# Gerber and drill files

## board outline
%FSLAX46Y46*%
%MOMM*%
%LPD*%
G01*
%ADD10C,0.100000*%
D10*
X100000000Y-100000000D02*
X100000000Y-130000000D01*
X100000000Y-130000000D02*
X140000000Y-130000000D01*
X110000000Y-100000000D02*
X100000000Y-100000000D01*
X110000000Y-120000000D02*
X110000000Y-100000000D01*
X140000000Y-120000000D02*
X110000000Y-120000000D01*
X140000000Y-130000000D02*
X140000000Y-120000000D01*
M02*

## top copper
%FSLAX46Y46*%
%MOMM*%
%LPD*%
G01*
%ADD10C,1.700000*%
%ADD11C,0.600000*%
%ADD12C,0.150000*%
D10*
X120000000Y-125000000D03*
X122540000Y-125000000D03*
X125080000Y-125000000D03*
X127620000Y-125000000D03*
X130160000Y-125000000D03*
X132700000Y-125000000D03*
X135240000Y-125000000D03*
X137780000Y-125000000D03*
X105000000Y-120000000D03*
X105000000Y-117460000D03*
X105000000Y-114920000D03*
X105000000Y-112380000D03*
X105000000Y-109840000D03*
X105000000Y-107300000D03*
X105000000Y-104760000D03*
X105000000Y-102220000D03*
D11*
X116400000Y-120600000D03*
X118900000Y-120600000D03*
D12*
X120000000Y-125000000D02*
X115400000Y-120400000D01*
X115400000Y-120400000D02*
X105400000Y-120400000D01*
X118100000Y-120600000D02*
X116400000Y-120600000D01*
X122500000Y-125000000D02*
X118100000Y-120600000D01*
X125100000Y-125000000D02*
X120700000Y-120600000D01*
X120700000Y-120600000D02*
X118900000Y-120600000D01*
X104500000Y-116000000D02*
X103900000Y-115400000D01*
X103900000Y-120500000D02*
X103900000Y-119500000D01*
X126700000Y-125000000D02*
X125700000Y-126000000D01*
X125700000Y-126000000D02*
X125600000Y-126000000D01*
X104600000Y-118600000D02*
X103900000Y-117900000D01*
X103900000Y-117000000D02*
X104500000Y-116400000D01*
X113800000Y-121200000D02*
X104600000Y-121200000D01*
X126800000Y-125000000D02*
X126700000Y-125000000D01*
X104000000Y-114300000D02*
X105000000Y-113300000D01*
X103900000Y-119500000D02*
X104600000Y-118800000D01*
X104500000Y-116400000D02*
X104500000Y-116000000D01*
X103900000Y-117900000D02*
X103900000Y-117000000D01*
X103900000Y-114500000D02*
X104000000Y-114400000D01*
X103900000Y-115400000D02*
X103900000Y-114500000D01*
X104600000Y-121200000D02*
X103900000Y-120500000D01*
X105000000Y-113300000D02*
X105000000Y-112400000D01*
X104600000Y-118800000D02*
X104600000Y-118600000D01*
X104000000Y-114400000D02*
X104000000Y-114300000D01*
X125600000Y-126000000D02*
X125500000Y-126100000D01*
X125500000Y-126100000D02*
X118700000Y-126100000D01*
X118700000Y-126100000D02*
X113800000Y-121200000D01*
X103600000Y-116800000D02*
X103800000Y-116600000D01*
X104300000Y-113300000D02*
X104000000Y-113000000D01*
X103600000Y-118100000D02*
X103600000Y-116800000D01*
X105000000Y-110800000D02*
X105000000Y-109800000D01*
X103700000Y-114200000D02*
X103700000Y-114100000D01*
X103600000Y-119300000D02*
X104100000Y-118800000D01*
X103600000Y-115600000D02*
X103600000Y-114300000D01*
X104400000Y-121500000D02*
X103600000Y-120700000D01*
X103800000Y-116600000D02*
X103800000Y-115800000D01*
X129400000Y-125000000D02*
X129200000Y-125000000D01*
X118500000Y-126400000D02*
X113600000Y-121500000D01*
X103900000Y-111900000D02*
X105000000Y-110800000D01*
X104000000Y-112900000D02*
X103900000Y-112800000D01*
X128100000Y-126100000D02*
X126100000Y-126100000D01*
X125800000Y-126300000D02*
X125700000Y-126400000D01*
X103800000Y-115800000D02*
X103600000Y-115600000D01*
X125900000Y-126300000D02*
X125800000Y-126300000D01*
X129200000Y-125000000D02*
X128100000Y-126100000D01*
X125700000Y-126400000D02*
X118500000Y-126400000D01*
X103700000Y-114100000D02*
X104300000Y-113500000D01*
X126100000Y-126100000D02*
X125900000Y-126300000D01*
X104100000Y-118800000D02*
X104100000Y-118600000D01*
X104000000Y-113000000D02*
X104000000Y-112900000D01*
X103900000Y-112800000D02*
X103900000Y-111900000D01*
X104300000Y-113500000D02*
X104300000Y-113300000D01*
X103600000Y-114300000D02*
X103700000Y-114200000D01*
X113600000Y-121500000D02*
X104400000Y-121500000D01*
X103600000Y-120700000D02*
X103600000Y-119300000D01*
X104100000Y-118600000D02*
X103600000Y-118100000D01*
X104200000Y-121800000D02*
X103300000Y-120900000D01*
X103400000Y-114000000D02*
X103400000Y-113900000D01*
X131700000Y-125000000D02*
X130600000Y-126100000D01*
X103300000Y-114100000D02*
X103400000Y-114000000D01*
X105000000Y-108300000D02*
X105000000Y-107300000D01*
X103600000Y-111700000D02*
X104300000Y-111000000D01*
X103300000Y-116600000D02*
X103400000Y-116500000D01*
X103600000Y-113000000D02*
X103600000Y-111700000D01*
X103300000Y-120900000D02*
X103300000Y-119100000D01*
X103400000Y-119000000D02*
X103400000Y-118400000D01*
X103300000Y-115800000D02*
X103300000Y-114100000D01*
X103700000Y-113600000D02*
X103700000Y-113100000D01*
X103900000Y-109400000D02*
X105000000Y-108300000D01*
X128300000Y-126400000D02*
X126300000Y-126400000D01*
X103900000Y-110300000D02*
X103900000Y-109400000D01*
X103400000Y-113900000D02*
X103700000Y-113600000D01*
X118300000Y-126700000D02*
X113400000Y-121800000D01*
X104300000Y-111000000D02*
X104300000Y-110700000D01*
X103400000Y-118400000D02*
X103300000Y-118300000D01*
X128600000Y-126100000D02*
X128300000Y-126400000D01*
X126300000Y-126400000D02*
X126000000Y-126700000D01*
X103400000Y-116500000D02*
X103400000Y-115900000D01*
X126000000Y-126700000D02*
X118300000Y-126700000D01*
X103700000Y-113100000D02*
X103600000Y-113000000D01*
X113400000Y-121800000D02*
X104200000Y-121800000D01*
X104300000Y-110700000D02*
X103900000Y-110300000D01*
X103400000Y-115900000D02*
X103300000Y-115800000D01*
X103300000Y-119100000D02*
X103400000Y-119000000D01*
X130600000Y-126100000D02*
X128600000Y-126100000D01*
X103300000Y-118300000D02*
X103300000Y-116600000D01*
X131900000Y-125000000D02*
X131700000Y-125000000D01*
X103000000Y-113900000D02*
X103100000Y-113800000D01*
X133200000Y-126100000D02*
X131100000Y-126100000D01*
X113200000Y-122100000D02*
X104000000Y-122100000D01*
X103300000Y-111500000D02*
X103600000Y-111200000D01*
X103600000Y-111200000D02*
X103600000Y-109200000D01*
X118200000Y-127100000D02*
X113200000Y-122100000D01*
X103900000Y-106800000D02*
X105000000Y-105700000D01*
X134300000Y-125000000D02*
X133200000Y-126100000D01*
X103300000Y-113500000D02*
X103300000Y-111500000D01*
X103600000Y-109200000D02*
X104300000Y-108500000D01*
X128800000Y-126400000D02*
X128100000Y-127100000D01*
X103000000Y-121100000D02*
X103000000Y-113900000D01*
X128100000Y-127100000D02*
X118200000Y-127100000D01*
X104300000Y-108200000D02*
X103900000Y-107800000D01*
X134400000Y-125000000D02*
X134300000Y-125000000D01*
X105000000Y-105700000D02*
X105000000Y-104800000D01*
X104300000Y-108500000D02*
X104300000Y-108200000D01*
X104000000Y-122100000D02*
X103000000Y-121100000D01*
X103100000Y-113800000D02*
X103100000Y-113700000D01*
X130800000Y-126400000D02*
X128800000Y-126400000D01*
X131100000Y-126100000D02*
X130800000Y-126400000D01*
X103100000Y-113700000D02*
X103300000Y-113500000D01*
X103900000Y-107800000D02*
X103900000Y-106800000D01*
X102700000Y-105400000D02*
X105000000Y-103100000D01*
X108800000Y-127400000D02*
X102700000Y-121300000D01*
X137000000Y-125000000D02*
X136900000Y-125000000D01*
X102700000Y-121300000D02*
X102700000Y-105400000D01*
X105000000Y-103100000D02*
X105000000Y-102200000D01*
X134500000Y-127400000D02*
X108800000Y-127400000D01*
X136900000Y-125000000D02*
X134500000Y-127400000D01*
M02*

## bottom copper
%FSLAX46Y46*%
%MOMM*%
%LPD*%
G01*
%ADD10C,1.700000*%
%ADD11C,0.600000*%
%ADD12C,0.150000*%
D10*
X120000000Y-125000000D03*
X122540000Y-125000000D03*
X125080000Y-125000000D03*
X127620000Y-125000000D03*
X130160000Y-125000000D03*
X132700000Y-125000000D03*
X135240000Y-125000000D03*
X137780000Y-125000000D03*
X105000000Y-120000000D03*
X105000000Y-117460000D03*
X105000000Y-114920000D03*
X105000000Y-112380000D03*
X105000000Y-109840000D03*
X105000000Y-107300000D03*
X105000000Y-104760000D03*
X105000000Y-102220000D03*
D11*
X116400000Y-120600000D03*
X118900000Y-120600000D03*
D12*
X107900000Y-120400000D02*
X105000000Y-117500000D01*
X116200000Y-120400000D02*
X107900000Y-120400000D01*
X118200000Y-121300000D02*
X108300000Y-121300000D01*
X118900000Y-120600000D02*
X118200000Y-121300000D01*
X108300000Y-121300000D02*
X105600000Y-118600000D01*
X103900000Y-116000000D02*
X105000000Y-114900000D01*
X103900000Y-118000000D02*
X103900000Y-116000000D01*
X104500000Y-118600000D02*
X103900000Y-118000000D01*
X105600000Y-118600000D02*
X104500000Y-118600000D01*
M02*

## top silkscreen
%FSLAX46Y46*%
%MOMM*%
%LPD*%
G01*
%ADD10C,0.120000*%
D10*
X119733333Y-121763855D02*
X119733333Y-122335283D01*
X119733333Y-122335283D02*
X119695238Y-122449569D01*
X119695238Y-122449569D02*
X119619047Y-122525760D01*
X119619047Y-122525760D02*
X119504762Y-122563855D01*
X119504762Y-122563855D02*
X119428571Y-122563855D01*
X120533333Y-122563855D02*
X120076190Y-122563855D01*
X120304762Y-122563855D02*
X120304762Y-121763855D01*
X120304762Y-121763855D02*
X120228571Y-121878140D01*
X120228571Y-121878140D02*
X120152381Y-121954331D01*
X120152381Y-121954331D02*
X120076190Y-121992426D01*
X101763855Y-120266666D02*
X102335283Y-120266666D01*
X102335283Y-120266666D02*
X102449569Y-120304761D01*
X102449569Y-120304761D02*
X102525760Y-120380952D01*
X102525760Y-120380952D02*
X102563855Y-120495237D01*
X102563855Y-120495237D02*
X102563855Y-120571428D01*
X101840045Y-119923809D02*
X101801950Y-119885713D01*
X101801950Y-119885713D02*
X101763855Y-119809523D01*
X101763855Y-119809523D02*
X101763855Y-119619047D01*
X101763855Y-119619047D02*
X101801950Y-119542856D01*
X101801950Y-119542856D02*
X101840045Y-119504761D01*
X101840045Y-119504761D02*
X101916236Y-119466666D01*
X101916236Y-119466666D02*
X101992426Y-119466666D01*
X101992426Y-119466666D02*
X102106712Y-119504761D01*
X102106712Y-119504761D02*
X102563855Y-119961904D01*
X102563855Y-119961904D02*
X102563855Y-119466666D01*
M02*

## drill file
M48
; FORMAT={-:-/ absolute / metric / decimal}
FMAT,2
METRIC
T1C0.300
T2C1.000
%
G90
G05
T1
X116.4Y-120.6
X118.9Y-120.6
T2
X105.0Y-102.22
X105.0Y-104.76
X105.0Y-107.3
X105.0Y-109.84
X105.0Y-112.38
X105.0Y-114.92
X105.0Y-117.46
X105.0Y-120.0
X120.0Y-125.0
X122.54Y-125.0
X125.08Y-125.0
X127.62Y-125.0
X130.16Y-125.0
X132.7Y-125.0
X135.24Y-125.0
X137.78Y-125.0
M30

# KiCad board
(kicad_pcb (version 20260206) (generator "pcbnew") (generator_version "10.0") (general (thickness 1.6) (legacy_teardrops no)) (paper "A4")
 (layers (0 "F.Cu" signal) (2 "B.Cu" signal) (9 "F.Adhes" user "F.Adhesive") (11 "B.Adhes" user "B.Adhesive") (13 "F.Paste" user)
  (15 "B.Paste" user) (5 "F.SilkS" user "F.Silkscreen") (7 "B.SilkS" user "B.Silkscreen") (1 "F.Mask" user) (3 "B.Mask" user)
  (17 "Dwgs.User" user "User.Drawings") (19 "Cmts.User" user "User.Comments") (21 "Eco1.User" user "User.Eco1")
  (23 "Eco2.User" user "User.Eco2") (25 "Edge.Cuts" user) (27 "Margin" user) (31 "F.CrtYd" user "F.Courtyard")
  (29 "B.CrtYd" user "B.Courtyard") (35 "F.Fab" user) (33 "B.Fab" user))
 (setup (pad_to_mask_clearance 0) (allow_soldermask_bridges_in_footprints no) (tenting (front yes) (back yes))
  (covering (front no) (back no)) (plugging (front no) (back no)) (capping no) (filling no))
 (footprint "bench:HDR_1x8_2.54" (layer "F.Cu") (at 120 125)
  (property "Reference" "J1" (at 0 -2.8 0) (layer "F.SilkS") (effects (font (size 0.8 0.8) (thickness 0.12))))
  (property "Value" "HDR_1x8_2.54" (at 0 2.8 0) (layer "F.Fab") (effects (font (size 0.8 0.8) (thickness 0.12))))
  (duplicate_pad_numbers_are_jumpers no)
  (pad "1" thru_hole circle (at 0 0) (size 1.7 1.7) (drill 1) (layers "*.Cu" "*.Mask") (remove_unused_layers no) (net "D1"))
  (pad "2" thru_hole circle (at 2.54 0) (size 1.7 1.7) (drill 1) (layers "*.Cu" "*.Mask") (remove_unused_layers no) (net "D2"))
  (pad "3" thru_hole circle (at 5.08 0) (size 1.7 1.7) (drill 1) (layers "*.Cu" "*.Mask") (remove_unused_layers no) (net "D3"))
  (pad "4" thru_hole circle (at 7.62 0) (size 1.7 1.7) (drill 1) (layers "*.Cu" "*.Mask") (remove_unused_layers no) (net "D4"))
  (pad "5" thru_hole circle (at 10.16 0) (size 1.7 1.7) (drill 1) (layers "*.Cu" "*.Mask") (remove_unused_layers no) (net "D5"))
  (pad "6" thru_hole circle (at 12.7 0) (size 1.7 1.7) (drill 1) (layers "*.Cu" "*.Mask") (remove_unused_layers no) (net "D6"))
  (pad "7" thru_hole circle (at 15.24 0) (size 1.7 1.7) (drill 1) (layers "*.Cu" "*.Mask") (remove_unused_layers no) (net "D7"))
  (pad "8" thru_hole circle (at 17.78 0) (size 1.7 1.7) (drill 1) (layers "*.Cu" "*.Mask") (remove_unused_layers no) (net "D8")))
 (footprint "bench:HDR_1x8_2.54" (layer "F.Cu") (at 105 120 90)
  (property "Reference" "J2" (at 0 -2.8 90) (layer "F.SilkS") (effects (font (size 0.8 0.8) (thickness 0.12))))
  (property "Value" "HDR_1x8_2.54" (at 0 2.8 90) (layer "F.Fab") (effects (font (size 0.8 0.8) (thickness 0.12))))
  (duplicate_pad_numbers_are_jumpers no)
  (pad "1" thru_hole circle (at 0 0 90) (size 1.7 1.7) (drill 1) (layers "*.Cu" "*.Mask") (remove_unused_layers no) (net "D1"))
  (pad "2" thru_hole circle (at 2.54 0 90) (size 1.7 1.7) (drill 1) (layers "*.Cu" "*.Mask") (remove_unused_layers no) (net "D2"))
  (pad "3" thru_hole circle (at 5.08 0 90) (size 1.7 1.7) (drill 1) (layers "*.Cu" "*.Mask") (remove_unused_layers no) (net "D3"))
  (pad "4" thru_hole circle (at 7.62 0 90) (size 1.7 1.7) (drill 1) (layers "*.Cu" "*.Mask") (remove_unused_layers no) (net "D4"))
  (pad "5" thru_hole circle (at 10.16 0 90) (size 1.7 1.7) (drill 1) (layers "*.Cu" "*.Mask") (remove_unused_layers no) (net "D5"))
  (pad "6" thru_hole circle (at 12.7 0 90) (size 1.7 1.7) (drill 1) (layers "*.Cu" "*.Mask") (remove_unused_layers no) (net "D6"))
  (pad "7" thru_hole circle (at 15.24 0 90) (size 1.7 1.7) (drill 1) (layers "*.Cu" "*.Mask") (remove_unused_layers no) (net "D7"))
  (pad "8" thru_hole circle (at 17.78 0 90) (size 1.7 1.7) (drill 1) (layers "*.Cu" "*.Mask") (remove_unused_layers no) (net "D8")))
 (gr_line (start 100 100) (end 100 130) (stroke (width 0.1) (type solid)) (layer "Edge.Cuts"))
 (gr_line (start 100 130) (end 140 130) (stroke (width 0.1) (type solid)) (layer "Edge.Cuts"))
 (gr_line (start 110 100) (end 100 100) (stroke (width 0.1) (type solid)) (layer "Edge.Cuts"))
 (gr_line (start 110 120) (end 110 100) (stroke (width 0.1) (type solid)) (layer "Edge.Cuts"))
 (gr_line (start 140 120) (end 110 120) (stroke (width 0.1) (type solid)) (layer "Edge.Cuts"))
 (gr_line (start 140 130) (end 140 120) (stroke (width 0.1) (type solid)) (layer "Edge.Cuts"))
 (segment (start 120 125) (end 115.4 120.4) (width 0.15) (layer "F.Cu") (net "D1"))
 (segment (start 115.4 120.4) (end 105.4 120.4) (width 0.15) (layer "F.Cu") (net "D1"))
 (segment (start 118.1 120.6) (end 116.4 120.6) (width 0.15) (layer "F.Cu") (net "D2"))
 (segment (start 122.5 125) (end 118.1 120.6) (width 0.15) (layer "F.Cu") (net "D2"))
 (via (at 116.4 120.6) (size 0.6) (drill 0.3) (layers "F.Cu" "B.Cu") (capping no) (covering (front no) (back no))
  (plugging (front no) (back no)) (filling no) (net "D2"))
 (segment (start 107.9 120.4) (end 105 117.5) (width 0.15) (layer "B.Cu") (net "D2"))
 (segment (start 116.2 120.4) (end 107.9 120.4) (width 0.15) (layer "B.Cu") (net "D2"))
 (segment (start 125.1 125) (end 120.7 120.6) (width 0.15) (layer "F.Cu") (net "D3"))
 (segment (start 120.7 120.6) (end 118.9 120.6) (width 0.15) (layer "F.Cu") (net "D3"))
 (via (at 118.9 120.6) (size 0.6) (drill 0.3) (layers "F.Cu" "B.Cu") (capping no) (covering (front no) (back no))
  (plugging (front no) (back no)) (filling no) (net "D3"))
 (segment (start 118.2 121.3) (end 108.3 121.3) (width 0.15) (layer "B.Cu") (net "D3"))
 (segment (start 118.9 120.6) (end 118.2 121.3) (width 0.15) (layer "B.Cu") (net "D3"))
 (segment (start 108.3 121.3) (end 105.6 118.6) (width 0.15) (layer "B.Cu") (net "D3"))
 (segment (start 103.9 116) (end 105 114.9) (width 0.15) (layer "B.Cu") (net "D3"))
 (segment (start 103.9 118) (end 103.9 116) (width 0.15) (layer "B.Cu") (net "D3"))
 (segment (start 104.5 118.6) (end 103.9 118) (width 0.15) (layer "B.Cu") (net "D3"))
 (segment (start 105.6 118.6) (end 104.5 118.6) (width 0.15) (layer "B.Cu") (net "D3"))
 (segment (start 104.5 116) (end 103.9 115.4) (width 0.15) (layer "F.Cu") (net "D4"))
 (segment (start 103.9 120.5) (end 103.9 119.5) (width 0.15) (layer "F.Cu") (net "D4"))
 (segment (start 126.7 125) (end 125.7 126) (width 0.15) (layer "F.Cu") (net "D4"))
 (segment (start 125.7 126) (end 125.6 126) (width 0.15) (layer "F.Cu") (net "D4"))
 (segment (start 104.6 118.6) (end 103.9 117.9) (width 0.15) (layer "F.Cu") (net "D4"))
 (segment (start 103.9 117) (end 104.5 116.4) (width 0.15) (layer "F.Cu") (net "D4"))
 (segment (start 113.8 121.2) (end 104.6 121.2) (width 0.15) (layer "F.Cu") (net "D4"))
 (segment (start 126.8 125) (end 126.7 125) (width 0.15) (layer "F.Cu") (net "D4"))
 (segment (start 104 114.3) (end 105 113.3) (width 0.15) (layer "F.Cu") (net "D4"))
 (segment (start 103.9 119.5) (end 104.6 118.8) (width 0.15) (layer "F.Cu") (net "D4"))
 (segment (start 104.5 116.4) (end 104.5 116) (width 0.15) (layer "F.Cu") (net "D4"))
 (segment (start 103.9 117.9) (end 103.9 117) (width 0.15) (layer "F.Cu") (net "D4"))
 (segment (start 103.9 114.5) (end 104 114.4) (width 0.15) (layer "F.Cu") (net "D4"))
 (segment (start 103.9 115.4) (end 103.9 114.5) (width 0.15) (layer "F.Cu") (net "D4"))
 (segment (start 104.6 121.2) (end 103.9 120.5) (width 0.15) (layer "F.Cu") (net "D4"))
 (segment (start 105 113.3) (end 105 112.4) (width 0.15) (layer "F.Cu") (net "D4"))
 (segment (start 104.6 118.8) (end 104.6 118.6) (width 0.15) (layer "F.Cu") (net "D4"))
 (segment (start 104 114.4) (end 104 114.3) (width 0.15) (layer "F.Cu") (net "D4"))
 (segment (start 125.6 126) (end 125.5 126.1) (width 0.15) (layer "F.Cu") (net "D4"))
 (segment (start 125.5 126.1) (end 118.7 126.1) (width 0.15) (layer "F.Cu") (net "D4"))
 (segment (start 118.7 126.1) (end 113.8 121.2) (width 0.15) (layer "F.Cu") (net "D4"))
 (segment (start 103.6 116.8) (end 103.8 116.6) (width 0.15) (layer "F.Cu") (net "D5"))
 (segment (start 104.3 113.3) (end 104 113) (width 0.15) (layer "F.Cu") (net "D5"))
 (segment (start 103.6 118.1) (end 103.6 116.8) (width 0.15) (layer "F.Cu") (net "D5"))
 (segment (start 105 110.8) (end 105 109.8) (width 0.15) (layer "F.Cu") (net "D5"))
 (segment (start 103.7 114.2) (end 103.7 114.1) (width 0.15) (layer "F.Cu") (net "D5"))
 (segment (start 103.6 119.3) (end 104.1 118.8) (width 0.15) (layer "F.Cu") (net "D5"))
 (segment (start 103.6 115.6) (end 103.6 114.3) (width 0.15) (layer "F.Cu") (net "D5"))
 (segment (start 104.4 121.5) (end 103.6 120.7) (width 0.15) (layer "F.Cu") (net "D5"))
 (segment (start 103.8 116.6) (end 103.8 115.8) (width 0.15) (layer "F.Cu") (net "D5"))
 (segment (start 129.4 125) (end 129.2 125) (width 0.15) (layer "F.Cu") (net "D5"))
 (segment (start 118.5 126.4) (end 113.6 121.5) (width 0.15) (layer "F.Cu") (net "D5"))
 (segment (start 103.9 111.9) (end 105 110.8) (width 0.15) (layer "F.Cu") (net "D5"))
 (segment (start 104 112.9) (end 103.9 112.8) (width 0.15) (layer "F.Cu") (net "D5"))
 (segment (start 128.1 126.1) (end 126.1 126.1) (width 0.15) (layer "F.Cu") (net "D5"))
 (segment (start 125.8 126.3) (end 125.7 126.4) (width 0.15) (layer "F.Cu") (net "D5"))
 (segment (start 103.8 115.8) (end 103.6 115.6) (width 0.15) (layer "F.Cu") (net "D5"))
 (segment (start 125.9 126.3) (end 125.8 126.3) (width 0.15) (layer "F.Cu") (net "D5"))
 (segment (start 129.2 125) (end 128.1 126.1) (width 0.15) (layer "F.Cu") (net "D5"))
 (segment (start 125.7 126.4) (end 118.5 126.4) (width 0.15) (layer "F.Cu") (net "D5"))
 (segment (start 103.7 114.1) (end 104.3 113.5) (width 0.15) (layer "F.Cu") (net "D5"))
 (segment (start 126.1 126.1) (end 125.9 126.3) (width 0.15) (layer "F.Cu") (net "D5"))
 (segment (start 104.1 118.8) (end 104.1 118.6) (width 0.15) (layer "F.Cu") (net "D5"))
 (segment (start 104 113) (end 104 112.9) (width 0.15) (layer "F.Cu") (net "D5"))
 (segment (start 103.9 112.8) (end 103.9 111.9) (width 0.15) (layer "F.Cu") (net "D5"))
 (segment (start 104.3 113.5) (end 104.3 113.3) (width 0.15) (layer "F.Cu") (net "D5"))
 (segment (start 103.6 114.3) (end 103.7 114.2) (width 0.15) (layer "F.Cu") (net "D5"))
 (segment (start 113.6 121.5) (end 104.4 121.5) (width 0.15) (layer "F.Cu") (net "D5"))
 (segment (start 103.6 120.7) (end 103.6 119.3) (width 0.15) (layer "F.Cu") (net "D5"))
 (segment (start 104.1 118.6) (end 103.6 118.1) (width 0.15) (layer "F.Cu") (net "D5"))
 (segment (start 104.2 121.8) (end 103.3 120.9) (width 0.15) (layer "F.Cu") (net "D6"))
 (segment (start 103.4 114) (end 103.4 113.9) (width 0.15) (layer "F.Cu") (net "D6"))
 (segment (start 131.7 125) (end 130.6 126.1) (width 0.15) (layer "F.Cu") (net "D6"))
 (segment (start 103.3 114.1) (end 103.4 114) (width 0.15) (layer "F.Cu") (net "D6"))
 (segment (start 105 108.3) (end 105 107.3) (width 0.15) (layer "F.Cu") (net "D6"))
 (segment (start 103.6 111.7) (end 104.3 111) (width 0.15) (layer "F.Cu") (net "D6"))
 (segment (start 103.3 116.6) (end 103.4 116.5) (width 0.15) (layer "F.Cu") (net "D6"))
 (segment (start 103.6 113) (end 103.6 111.7) (width 0.15) (layer "F.Cu") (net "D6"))
 (segment (start 103.3 120.9) (end 103.3 119.1) (width 0.15) (layer "F.Cu") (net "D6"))
 (segment (start 103.4 119) (end 103.4 118.4) (width 0.15) (layer "F.Cu") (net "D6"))
 (segment (start 103.3 115.8) (end 103.3 114.1) (width 0.15) (layer "F.Cu") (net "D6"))
 (segment (start 103.7 113.6) (end 103.7 113.1) (width 0.15) (layer "F.Cu") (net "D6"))
 (segment (start 103.9 109.4) (end 105 108.3) (width 0.15) (layer "F.Cu") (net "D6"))
 (segment (start 128.3 126.4) (end 126.3 126.4) (width 0.15) (layer "F.Cu") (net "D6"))
 (segment (start 103.9 110.3) (end 103.9 109.4) (width 0.15) (layer "F.Cu") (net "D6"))
 (segment (start 103.4 113.9) (end 103.7 113.6) (width 0.15) (layer "F.Cu") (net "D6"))
 (segment (start 118.3 126.7) (end 113.4 121.8) (width 0.15) (layer "F.Cu") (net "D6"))
 (segment (start 104.3 111) (end 104.3 110.7) (width 0.15) (layer "F.Cu") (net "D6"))
 (segment (start 103.4 118.4) (end 103.3 118.3) (width 0.15) (layer "F.Cu") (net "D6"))
 (segment (start 128.6 126.1) (end 128.3 126.4) (width 0.15) (layer "F.Cu") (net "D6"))
 (segment (start 126.3 126.4) (end 126 126.7) (width 0.15) (layer "F.Cu") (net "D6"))
 (segment (start 103.4 116.5) (end 103.4 115.9) (width 0.15) (layer "F.Cu") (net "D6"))
 (segment (start 126 126.7) (end 118.3 126.7) (width 0.15) (layer "F.Cu") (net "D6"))
 (segment (start 103.7 113.1) (end 103.6 113) (width 0.15) (layer "F.Cu") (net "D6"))
 (segment (start 113.4 121.8) (end 104.2 121.8) (width 0.15) (layer "F.Cu") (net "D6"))
 (segment (start 104.3 110.7) (end 103.9 110.3) (width 0.15) (layer "F.Cu") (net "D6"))
 (segment (start 103.4 115.9) (end 103.3 115.8) (width 0.15) (layer "F.Cu") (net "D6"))
 (segment (start 103.3 119.1) (end 103.4 119) (width 0.15) (layer "F.Cu") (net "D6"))
 (segment (start 130.6 126.1) (end 128.6 126.1) (width 0.15) (layer "F.Cu") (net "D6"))
 (segment (start 103.3 118.3) (end 103.3 116.6) (width 0.15) (layer "F.Cu") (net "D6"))
 (segment (start 131.9 125) (end 131.7 125) (width 0.15) (layer "F.Cu") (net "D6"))
 (segment (start 103 113.9) (end 103.1 113.8) (width 0.15) (layer "F.Cu") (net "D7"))
 (segment (start 133.2 126.1) (end 131.1 126.1) (width 0.15) (layer "F.Cu") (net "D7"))
 (segment (start 113.2 122.1) (end 104 122.1) (width 0.15) (layer "F.Cu") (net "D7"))
 (segment (start 103.3 111.5) (end 103.6 111.2) (width 0.15) (layer "F.Cu") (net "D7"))
 (segment (start 103.6 111.2) (end 103.6 109.2) (width 0.15) (layer "F.Cu") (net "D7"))
 (segment (start 118.2 127.1) (end 113.2 122.1) (width 0.15) (layer "F.Cu") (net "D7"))
 (segment (start 103.9 106.8) (end 105 105.7) (width 0.15) (layer "F.Cu") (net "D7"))
 (segment (start 134.3 125) (end 133.2 126.1) (width 0.15) (layer "F.Cu") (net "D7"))
 (segment (start 103.3 113.5) (end 103.3 111.5) (width 0.15) (layer "F.Cu") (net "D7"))
 (segment (start 103.6 109.2) (end 104.3 108.5) (width 0.15) (layer "F.Cu") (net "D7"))
 (segment (start 128.8 126.4) (end 128.1 127.1) (width 0.15) (layer "F.Cu") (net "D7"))
 (segment (start 103 121.1) (end 103 113.9) (width 0.15) (layer "F.Cu") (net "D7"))
 (segment (start 128.1 127.1) (end 118.2 127.1) (width 0.15) (layer "F.Cu") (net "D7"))
 (segment (start 104.3 108.2) (end 103.9 107.8) (width 0.15) (layer "F.Cu") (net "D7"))
 (segment (start 134.4 125) (end 134.3 125) (width 0.15) (layer "F.Cu") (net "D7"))
 (segment (start 105 105.7) (end 105 104.8) (width 0.15) (layer "F.Cu") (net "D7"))
 (segment (start 104.3 108.5) (end 104.3 108.2) (width 0.15) (layer "F.Cu") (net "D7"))
 (segment (start 104 122.1) (end 103 121.1) (width 0.15) (layer "F.Cu") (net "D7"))
 (segment (start 103.1 113.8) (end 103.1 113.7) (width 0.15) (layer "F.Cu") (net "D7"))
 (segment (start 130.8 126.4) (end 128.8 126.4) (width 0.15) (layer "F.Cu") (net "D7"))
 (segment (start 131.1 126.1) (end 130.8 126.4) (width 0.15) (layer "F.Cu") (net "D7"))
 (segment (start 103.1 113.7) (end 103.3 113.5) (width 0.15) (layer "F.Cu") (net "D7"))
 (segment (start 103.9 107.8) (end 103.9 106.8) (width 0.15) (layer "F.Cu") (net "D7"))
 (segment (start 102.7 105.4) (end 105 103.1) (width 0.15) (layer "F.Cu") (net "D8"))
 (segment (start 108.8 127.4) (end 102.7 121.3) (width 0.15) (layer "F.Cu") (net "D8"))
 (segment (start 137 125) (end 136.9 125) (width 0.15) (layer "F.Cu") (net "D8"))
 (segment (start 102.7 121.3) (end 102.7 105.4) (width 0.15) (layer "F.Cu") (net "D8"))
 (segment (start 105 103.1) (end 105 102.2) (width 0.15) (layer "F.Cu") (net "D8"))
 (segment (start 134.5 127.4) (end 108.8 127.4) (width 0.15) (layer "F.Cu") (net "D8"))
 (segment (start 136.9 125) (end 134.5 127.4) (width 0.15) (layer "F.Cu") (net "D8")))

